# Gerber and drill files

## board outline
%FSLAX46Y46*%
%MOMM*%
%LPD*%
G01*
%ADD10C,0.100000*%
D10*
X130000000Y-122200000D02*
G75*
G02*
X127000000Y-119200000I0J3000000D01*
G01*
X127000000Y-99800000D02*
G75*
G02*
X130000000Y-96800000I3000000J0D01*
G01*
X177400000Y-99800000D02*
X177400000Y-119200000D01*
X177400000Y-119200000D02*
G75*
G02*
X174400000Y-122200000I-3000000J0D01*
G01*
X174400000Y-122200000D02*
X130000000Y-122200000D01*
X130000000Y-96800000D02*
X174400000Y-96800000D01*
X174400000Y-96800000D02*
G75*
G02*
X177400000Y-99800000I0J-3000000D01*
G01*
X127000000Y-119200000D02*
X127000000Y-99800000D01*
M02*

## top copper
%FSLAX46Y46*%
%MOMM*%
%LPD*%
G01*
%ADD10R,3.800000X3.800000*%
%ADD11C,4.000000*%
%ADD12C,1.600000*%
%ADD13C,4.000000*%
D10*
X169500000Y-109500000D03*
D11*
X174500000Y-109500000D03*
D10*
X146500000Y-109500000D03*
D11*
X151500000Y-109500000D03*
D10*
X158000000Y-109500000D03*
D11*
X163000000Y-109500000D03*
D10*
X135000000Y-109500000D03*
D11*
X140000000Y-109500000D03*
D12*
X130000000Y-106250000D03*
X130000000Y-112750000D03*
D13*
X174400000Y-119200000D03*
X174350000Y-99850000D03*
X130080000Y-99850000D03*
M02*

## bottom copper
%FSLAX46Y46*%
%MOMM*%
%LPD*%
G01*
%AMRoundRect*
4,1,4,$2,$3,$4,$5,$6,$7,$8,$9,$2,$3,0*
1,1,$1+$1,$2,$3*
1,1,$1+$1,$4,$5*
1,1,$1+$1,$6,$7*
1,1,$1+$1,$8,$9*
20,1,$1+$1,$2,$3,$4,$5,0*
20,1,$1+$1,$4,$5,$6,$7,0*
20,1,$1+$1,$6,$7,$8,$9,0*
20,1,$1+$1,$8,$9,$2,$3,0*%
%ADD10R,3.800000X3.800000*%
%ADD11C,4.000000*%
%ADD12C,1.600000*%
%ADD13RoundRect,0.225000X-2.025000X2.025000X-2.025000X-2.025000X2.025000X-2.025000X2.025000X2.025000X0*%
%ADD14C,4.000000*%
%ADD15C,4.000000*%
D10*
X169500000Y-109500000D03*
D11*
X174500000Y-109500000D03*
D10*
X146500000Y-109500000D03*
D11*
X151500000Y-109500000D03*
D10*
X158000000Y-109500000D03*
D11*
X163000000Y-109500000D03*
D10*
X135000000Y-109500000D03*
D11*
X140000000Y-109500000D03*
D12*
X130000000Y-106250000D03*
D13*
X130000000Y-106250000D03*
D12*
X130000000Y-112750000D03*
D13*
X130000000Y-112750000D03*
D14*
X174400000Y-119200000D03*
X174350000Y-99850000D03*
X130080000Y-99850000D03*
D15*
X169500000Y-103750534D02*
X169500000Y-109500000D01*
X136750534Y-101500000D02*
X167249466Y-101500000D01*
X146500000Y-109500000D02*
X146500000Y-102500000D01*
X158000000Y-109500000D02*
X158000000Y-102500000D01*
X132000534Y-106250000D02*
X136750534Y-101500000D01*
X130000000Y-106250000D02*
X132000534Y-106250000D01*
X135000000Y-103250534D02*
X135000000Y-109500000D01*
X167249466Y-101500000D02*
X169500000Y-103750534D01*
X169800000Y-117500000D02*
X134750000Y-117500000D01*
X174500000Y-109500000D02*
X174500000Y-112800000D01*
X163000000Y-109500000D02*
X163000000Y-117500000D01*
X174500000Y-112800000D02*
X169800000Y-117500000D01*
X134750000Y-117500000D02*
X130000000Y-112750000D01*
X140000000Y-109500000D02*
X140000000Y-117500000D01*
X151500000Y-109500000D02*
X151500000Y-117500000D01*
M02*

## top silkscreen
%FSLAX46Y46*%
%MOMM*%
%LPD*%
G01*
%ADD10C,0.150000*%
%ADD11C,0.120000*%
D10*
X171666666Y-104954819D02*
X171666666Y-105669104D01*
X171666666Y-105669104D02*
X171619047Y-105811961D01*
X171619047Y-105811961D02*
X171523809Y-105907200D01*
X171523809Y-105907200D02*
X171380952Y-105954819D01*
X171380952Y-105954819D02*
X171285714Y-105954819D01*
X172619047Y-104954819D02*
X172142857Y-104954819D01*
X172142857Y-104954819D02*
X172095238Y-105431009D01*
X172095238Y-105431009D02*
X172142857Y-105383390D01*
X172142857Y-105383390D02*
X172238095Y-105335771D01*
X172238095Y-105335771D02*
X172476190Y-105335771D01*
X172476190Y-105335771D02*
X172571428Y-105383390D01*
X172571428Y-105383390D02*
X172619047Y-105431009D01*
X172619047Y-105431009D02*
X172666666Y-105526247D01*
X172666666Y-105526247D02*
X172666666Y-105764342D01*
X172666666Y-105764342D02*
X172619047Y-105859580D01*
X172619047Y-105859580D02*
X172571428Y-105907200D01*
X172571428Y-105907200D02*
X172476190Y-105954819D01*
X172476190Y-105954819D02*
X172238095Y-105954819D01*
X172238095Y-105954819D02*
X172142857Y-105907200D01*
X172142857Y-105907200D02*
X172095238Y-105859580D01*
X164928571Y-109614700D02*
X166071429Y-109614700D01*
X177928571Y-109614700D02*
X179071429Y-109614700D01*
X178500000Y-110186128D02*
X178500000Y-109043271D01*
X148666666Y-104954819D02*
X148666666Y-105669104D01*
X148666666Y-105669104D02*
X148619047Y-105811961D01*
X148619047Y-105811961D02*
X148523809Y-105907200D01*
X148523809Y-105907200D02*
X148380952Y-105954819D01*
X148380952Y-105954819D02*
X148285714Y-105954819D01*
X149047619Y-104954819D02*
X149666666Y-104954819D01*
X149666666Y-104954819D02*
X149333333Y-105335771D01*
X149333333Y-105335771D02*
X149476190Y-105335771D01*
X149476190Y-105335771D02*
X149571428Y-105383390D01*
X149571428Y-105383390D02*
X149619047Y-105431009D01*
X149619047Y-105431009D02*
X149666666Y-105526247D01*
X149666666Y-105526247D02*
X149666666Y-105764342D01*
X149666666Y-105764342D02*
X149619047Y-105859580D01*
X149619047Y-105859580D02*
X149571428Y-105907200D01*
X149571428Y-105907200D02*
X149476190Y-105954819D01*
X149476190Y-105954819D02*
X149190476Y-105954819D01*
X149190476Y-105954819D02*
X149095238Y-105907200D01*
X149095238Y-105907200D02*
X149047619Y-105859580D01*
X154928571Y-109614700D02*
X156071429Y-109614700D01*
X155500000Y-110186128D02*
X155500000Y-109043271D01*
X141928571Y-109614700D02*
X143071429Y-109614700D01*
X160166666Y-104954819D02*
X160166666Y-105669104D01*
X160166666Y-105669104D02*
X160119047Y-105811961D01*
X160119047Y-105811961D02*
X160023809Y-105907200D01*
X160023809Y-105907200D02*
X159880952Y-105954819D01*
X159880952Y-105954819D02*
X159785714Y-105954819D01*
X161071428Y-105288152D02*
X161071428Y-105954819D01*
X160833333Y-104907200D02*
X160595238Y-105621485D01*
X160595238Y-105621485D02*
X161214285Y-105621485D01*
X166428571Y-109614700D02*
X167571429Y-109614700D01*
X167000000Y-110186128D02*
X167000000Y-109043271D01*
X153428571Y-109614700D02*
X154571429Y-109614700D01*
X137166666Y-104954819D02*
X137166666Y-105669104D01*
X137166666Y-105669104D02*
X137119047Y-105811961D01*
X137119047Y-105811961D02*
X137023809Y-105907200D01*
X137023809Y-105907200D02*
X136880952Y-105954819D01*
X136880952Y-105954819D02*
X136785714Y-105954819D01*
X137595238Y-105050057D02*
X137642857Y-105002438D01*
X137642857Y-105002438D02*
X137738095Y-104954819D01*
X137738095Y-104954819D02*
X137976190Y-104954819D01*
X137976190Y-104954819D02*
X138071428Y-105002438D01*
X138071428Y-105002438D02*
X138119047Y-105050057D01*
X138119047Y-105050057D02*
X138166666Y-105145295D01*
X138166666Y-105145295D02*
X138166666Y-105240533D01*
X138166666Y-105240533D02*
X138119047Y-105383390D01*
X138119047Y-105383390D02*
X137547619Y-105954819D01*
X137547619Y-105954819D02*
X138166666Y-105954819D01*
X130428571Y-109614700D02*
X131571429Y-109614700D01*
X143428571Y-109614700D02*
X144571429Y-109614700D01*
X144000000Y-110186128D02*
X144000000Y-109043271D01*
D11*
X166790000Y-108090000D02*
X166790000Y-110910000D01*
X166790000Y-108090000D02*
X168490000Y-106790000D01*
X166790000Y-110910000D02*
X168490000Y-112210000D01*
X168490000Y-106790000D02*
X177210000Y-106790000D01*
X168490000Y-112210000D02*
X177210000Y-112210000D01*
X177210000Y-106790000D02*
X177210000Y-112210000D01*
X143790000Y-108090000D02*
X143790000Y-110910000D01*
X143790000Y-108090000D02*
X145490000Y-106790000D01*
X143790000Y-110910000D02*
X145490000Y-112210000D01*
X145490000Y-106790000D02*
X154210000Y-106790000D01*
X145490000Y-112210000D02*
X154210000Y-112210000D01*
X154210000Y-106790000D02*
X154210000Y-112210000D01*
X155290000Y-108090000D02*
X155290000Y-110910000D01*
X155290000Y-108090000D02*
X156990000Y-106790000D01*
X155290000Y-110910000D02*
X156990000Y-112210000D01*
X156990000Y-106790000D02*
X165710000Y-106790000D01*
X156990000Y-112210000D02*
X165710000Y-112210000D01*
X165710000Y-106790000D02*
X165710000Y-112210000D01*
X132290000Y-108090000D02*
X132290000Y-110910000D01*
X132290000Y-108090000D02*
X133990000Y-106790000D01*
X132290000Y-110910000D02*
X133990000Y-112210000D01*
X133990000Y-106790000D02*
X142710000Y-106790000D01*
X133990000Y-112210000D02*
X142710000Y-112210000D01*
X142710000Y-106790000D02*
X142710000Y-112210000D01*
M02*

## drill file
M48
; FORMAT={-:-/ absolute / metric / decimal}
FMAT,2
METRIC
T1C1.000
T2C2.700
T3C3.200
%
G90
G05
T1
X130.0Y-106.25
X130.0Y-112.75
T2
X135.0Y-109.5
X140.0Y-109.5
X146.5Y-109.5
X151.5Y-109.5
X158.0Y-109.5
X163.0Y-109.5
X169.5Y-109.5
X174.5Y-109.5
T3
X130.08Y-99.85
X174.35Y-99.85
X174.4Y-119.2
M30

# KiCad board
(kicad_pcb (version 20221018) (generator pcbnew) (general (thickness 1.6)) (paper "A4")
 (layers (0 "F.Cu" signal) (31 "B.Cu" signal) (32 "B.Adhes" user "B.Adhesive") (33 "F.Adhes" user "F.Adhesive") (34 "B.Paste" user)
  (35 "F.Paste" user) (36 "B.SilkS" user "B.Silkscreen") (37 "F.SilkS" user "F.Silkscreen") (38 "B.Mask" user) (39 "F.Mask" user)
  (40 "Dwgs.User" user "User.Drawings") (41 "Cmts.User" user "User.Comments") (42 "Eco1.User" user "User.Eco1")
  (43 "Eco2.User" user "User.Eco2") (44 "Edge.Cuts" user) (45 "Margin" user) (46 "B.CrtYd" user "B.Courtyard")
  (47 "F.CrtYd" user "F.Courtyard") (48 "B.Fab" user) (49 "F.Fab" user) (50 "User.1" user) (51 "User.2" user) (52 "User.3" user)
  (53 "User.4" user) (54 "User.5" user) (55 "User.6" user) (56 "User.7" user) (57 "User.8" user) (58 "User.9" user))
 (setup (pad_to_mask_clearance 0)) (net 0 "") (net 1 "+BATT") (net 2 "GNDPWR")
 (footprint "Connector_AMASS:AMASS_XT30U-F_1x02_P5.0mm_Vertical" (layer "F.Cu") (at 169.5 109.5)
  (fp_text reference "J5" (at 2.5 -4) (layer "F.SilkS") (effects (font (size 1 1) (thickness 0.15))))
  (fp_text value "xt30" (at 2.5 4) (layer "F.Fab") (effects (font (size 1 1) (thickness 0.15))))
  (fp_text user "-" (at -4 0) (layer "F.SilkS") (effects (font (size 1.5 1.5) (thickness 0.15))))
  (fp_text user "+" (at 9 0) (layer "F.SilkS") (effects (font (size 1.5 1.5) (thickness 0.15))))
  (fp_line (start -2.71 -1.41) (end -2.71 1.41) (stroke (width 0.12) (type solid)) (layer "F.SilkS"))
  (fp_line (start -2.71 -1.41) (end -1.01 -2.71) (stroke (width 0.12) (type solid)) (layer "F.SilkS"))
  (fp_line (start -2.71 1.41) (end -1.01 2.71) (stroke (width 0.12) (type solid)) (layer "F.SilkS"))
  (fp_line (start -1.01 -2.71) (end 7.71 -2.71) (stroke (width 0.12) (type solid)) (layer "F.SilkS"))
  (fp_line (start -1.01 2.71) (end 7.71 2.71) (stroke (width 0.12) (type solid)) (layer "F.SilkS"))
  (fp_line (start 7.71 -2.71) (end 7.71 2.71) (stroke (width 0.12) (type solid)) (layer "F.SilkS"))
  (pad "1" thru_hole rect (at 0 0) (size 3.8 3.8) (drill 2.7) (layers "*.Cu" "*.Mask") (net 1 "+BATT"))
  (pad "2" thru_hole circle (at 5 0) (size 4 4) (drill 2.7) (layers "*.Cu" "*.Mask") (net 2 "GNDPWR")))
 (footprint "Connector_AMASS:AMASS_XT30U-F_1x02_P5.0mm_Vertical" (layer "F.Cu") (at 146.5 109.5)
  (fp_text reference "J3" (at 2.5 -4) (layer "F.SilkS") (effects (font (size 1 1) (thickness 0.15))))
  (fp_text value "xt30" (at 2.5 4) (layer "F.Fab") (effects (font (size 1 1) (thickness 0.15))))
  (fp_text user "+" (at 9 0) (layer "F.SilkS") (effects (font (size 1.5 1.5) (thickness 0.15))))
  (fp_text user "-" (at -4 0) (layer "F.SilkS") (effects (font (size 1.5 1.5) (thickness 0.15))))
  (fp_line (start -2.71 -1.41) (end -2.71 1.41) (stroke (width 0.12) (type solid)) (layer "F.SilkS"))
  (fp_line (start -2.71 -1.41) (end -1.01 -2.71) (stroke (width 0.12) (type solid)) (layer "F.SilkS"))
  (fp_line (start -2.71 1.41) (end -1.01 2.71) (stroke (width 0.12) (type solid)) (layer "F.SilkS"))
  (fp_line (start -1.01 -2.71) (end 7.71 -2.71) (stroke (width 0.12) (type solid)) (layer "F.SilkS"))
  (fp_line (start -1.01 2.71) (end 7.71 2.71) (stroke (width 0.12) (type solid)) (layer "F.SilkS"))
  (fp_line (start 7.71 -2.71) (end 7.71 2.71) (stroke (width 0.12) (type solid)) (layer "F.SilkS"))
  (pad "1" thru_hole rect (at 0 0) (size 3.8 3.8) (drill 2.7) (layers "*.Cu" "*.Mask") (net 1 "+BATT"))
  (pad "2" thru_hole circle (at 5 0) (size 4 4) (drill 2.7) (layers "*.Cu" "*.Mask") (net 2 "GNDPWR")))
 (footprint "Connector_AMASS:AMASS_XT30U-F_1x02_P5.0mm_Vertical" (layer "F.Cu") (at 158 109.5)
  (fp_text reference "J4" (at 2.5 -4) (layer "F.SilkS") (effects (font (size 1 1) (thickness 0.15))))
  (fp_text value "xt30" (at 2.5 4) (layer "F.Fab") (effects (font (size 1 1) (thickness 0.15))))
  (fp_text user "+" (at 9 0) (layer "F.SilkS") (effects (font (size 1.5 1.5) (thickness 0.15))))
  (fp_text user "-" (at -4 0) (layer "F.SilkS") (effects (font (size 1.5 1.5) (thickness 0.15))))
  (fp_line (start -2.71 -1.41) (end -2.71 1.41) (stroke (width 0.12) (type solid)) (layer "F.SilkS"))
  (fp_line (start -2.71 -1.41) (end -1.01 -2.71) (stroke (width 0.12) (type solid)) (layer "F.SilkS"))
  (fp_line (start -2.71 1.41) (end -1.01 2.71) (stroke (width 0.12) (type solid)) (layer "F.SilkS"))
  (fp_line (start -1.01 -2.71) (end 7.71 -2.71) (stroke (width 0.12) (type solid)) (layer "F.SilkS"))
  (fp_line (start -1.01 2.71) (end 7.71 2.71) (stroke (width 0.12) (type solid)) (layer "F.SilkS"))
  (fp_line (start 7.71 -2.71) (end 7.71 2.71) (stroke (width 0.12) (type solid)) (layer "F.SilkS"))
  (pad "1" thru_hole rect (at 0 0) (size 3.8 3.8) (drill 2.7) (layers "*.Cu" "*.Mask") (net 1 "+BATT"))
  (pad "2" thru_hole circle (at 5 0) (size 4 4) (drill 2.7) (layers "*.Cu" "*.Mask") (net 2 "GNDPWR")))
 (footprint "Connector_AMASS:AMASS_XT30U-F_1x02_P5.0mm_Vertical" (layer "F.Cu") (at 135 109.5)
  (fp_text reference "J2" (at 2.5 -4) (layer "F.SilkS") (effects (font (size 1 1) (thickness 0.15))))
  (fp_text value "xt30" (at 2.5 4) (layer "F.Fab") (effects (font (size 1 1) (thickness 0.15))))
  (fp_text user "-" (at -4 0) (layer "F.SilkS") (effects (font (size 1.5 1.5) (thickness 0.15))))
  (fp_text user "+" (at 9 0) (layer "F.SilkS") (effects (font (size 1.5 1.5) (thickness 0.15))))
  (fp_line (start -2.71 -1.41) (end -2.71 1.41) (stroke (width 0.12) (type solid)) (layer "F.SilkS"))
  (fp_line (start -2.71 -1.41) (end -1.01 -2.71) (stroke (width 0.12) (type solid)) (layer "F.SilkS"))
  (fp_line (start -2.71 1.41) (end -1.01 2.71) (stroke (width 0.12) (type solid)) (layer "F.SilkS"))
  (fp_line (start -1.01 -2.71) (end 7.71 -2.71) (stroke (width 0.12) (type solid)) (layer "F.SilkS"))
  (fp_line (start -1.01 2.71) (end 7.71 2.71) (stroke (width 0.12) (type solid)) (layer "F.SilkS"))
  (fp_line (start 7.71 -2.71) (end 7.71 2.71) (stroke (width 0.12) (type solid)) (layer "F.SilkS"))
  (pad "1" thru_hole rect (at 0 0) (size 3.8 3.8) (drill 2.7) (layers "*.Cu" "*.Mask") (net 1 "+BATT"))
  (pad "2" thru_hole circle (at 5 0) (size 4 4) (drill 2.7) (layers "*.Cu" "*.Mask") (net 2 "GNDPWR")))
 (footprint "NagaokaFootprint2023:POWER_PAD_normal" (layer "B.Cu") (at 130 109.5 -90)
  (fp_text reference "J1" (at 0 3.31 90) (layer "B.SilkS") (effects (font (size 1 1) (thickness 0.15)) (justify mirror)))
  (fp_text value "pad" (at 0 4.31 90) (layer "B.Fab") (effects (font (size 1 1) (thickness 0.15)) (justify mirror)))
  (pad "1" thru_hole circle (at -3.25 0 270) (size 1.6 1.6) (drill 1) (layers "*.Cu" "*.Mask") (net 1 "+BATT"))
  (pad "1" smd roundrect (at -3.25 0 270) (size 4.5 4.5) (layers "B.Cu" "B.Paste" "B.Mask") (roundrect_rratio 0.05) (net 1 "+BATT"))
  (pad "2" thru_hole circle (at 3.25 0 270) (size 1.6 1.6) (drill 1) (layers "*.Cu" "*.Mask") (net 2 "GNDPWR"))
  (pad "2" smd roundrect (at 3.25 0 270) (size 4.5 4.5) (layers "B.Cu" "B.Paste" "B.Mask") (roundrect_rratio 0.05) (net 2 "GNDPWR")))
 (gr_arc (start 130 122.2) (mid 127.87868 121.32132) (end 127 119.2) (stroke (width 0.1) (type default)) (layer "Edge.Cuts"))
 (gr_arc (start 127 99.8) (mid 127.87868 97.67868) (end 130 96.8) (stroke (width 0.1) (type default)) (layer "Edge.Cuts"))
 (gr_line (start 177.4 99.8) (end 177.4 119.2) (stroke (width 0.1) (type default)) (layer "Edge.Cuts"))
 (gr_arc (start 177.4 119.2) (mid 176.52132 121.32132) (end 174.4 122.2) (stroke (width 0.1) (type default)) (layer "Edge.Cuts"))
 (gr_line (start 174.4 122.2) (end 130 122.2) (stroke (width 0.1) (type default)) (layer "Edge.Cuts"))
 (gr_line (start 130 96.8) (end 174.4 96.8) (stroke (width 0.1) (type default)) (layer "Edge.Cuts"))
 (gr_arc (start 174.4 96.8) (mid 176.52132 97.67868) (end 177.4 99.8) (stroke (width 0.1) (type default)) (layer "Edge.Cuts"))
 (gr_line (start 127 119.2) (end 127 99.8) (stroke (width 0.1) (type default)) (layer "Edge.Cuts"))
 (via (at 174.4 119.2) (size 4) (drill 3.2) (layers "F.Cu" "B.Cu") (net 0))
 (via (at 174.35 99.85) (size 4) (drill 3.2) (layers "F.Cu" "B.Cu") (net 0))
 (via (at 130.08 99.85) (size 4) (drill 3.2) (layers "F.Cu" "B.Cu") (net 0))
 (segment (start 169.5 103.750534) (end 169.5 109.5) (width 4) (layer "B.Cu") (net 1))
 (segment (start 136.750534 101.5) (end 167.249466 101.5) (width 4) (layer "B.Cu") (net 1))
 (segment (start 146.5 109.5) (end 146.5 102.5) (width 4) (layer "B.Cu") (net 1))
 (segment (start 158 109.5) (end 158 102.5) (width 4) (layer "B.Cu") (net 1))
 (segment (start 132.000534 106.25) (end 136.750534 101.5) (width 4) (layer "B.Cu") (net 1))
 (segment (start 130 106.25) (end 132.000534 106.25) (width 4) (layer "B.Cu") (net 1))
 (segment (start 135 103.250534) (end 135 109.5) (width 4) (layer "B.Cu") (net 1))
 (segment (start 167.249466 101.5) (end 169.5 103.750534) (width 4) (layer "B.Cu") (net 1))
 (segment (start 169.8 117.5) (end 134.75 117.5) (width 4) (layer "B.Cu") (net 2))
 (segment (start 174.5 109.5) (end 174.5 112.8) (width 4) (layer "B.Cu") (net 2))
 (segment (start 163 109.5) (end 163 117.5) (width 4) (layer "B.Cu") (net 2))
 (segment (start 174.5 112.8) (end 169.8 117.5) (width 4) (layer "B.Cu") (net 2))
 (segment (start 134.75 117.5) (end 130 112.75) (width 4) (layer "B.Cu") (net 2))
 (segment (start 140 109.5) (end 140 117.5) (width 4) (layer "B.Cu") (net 2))
 (segment (start 151.5 109.5) (end 151.5 117.5) (width 4) (layer "B.Cu") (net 2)))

